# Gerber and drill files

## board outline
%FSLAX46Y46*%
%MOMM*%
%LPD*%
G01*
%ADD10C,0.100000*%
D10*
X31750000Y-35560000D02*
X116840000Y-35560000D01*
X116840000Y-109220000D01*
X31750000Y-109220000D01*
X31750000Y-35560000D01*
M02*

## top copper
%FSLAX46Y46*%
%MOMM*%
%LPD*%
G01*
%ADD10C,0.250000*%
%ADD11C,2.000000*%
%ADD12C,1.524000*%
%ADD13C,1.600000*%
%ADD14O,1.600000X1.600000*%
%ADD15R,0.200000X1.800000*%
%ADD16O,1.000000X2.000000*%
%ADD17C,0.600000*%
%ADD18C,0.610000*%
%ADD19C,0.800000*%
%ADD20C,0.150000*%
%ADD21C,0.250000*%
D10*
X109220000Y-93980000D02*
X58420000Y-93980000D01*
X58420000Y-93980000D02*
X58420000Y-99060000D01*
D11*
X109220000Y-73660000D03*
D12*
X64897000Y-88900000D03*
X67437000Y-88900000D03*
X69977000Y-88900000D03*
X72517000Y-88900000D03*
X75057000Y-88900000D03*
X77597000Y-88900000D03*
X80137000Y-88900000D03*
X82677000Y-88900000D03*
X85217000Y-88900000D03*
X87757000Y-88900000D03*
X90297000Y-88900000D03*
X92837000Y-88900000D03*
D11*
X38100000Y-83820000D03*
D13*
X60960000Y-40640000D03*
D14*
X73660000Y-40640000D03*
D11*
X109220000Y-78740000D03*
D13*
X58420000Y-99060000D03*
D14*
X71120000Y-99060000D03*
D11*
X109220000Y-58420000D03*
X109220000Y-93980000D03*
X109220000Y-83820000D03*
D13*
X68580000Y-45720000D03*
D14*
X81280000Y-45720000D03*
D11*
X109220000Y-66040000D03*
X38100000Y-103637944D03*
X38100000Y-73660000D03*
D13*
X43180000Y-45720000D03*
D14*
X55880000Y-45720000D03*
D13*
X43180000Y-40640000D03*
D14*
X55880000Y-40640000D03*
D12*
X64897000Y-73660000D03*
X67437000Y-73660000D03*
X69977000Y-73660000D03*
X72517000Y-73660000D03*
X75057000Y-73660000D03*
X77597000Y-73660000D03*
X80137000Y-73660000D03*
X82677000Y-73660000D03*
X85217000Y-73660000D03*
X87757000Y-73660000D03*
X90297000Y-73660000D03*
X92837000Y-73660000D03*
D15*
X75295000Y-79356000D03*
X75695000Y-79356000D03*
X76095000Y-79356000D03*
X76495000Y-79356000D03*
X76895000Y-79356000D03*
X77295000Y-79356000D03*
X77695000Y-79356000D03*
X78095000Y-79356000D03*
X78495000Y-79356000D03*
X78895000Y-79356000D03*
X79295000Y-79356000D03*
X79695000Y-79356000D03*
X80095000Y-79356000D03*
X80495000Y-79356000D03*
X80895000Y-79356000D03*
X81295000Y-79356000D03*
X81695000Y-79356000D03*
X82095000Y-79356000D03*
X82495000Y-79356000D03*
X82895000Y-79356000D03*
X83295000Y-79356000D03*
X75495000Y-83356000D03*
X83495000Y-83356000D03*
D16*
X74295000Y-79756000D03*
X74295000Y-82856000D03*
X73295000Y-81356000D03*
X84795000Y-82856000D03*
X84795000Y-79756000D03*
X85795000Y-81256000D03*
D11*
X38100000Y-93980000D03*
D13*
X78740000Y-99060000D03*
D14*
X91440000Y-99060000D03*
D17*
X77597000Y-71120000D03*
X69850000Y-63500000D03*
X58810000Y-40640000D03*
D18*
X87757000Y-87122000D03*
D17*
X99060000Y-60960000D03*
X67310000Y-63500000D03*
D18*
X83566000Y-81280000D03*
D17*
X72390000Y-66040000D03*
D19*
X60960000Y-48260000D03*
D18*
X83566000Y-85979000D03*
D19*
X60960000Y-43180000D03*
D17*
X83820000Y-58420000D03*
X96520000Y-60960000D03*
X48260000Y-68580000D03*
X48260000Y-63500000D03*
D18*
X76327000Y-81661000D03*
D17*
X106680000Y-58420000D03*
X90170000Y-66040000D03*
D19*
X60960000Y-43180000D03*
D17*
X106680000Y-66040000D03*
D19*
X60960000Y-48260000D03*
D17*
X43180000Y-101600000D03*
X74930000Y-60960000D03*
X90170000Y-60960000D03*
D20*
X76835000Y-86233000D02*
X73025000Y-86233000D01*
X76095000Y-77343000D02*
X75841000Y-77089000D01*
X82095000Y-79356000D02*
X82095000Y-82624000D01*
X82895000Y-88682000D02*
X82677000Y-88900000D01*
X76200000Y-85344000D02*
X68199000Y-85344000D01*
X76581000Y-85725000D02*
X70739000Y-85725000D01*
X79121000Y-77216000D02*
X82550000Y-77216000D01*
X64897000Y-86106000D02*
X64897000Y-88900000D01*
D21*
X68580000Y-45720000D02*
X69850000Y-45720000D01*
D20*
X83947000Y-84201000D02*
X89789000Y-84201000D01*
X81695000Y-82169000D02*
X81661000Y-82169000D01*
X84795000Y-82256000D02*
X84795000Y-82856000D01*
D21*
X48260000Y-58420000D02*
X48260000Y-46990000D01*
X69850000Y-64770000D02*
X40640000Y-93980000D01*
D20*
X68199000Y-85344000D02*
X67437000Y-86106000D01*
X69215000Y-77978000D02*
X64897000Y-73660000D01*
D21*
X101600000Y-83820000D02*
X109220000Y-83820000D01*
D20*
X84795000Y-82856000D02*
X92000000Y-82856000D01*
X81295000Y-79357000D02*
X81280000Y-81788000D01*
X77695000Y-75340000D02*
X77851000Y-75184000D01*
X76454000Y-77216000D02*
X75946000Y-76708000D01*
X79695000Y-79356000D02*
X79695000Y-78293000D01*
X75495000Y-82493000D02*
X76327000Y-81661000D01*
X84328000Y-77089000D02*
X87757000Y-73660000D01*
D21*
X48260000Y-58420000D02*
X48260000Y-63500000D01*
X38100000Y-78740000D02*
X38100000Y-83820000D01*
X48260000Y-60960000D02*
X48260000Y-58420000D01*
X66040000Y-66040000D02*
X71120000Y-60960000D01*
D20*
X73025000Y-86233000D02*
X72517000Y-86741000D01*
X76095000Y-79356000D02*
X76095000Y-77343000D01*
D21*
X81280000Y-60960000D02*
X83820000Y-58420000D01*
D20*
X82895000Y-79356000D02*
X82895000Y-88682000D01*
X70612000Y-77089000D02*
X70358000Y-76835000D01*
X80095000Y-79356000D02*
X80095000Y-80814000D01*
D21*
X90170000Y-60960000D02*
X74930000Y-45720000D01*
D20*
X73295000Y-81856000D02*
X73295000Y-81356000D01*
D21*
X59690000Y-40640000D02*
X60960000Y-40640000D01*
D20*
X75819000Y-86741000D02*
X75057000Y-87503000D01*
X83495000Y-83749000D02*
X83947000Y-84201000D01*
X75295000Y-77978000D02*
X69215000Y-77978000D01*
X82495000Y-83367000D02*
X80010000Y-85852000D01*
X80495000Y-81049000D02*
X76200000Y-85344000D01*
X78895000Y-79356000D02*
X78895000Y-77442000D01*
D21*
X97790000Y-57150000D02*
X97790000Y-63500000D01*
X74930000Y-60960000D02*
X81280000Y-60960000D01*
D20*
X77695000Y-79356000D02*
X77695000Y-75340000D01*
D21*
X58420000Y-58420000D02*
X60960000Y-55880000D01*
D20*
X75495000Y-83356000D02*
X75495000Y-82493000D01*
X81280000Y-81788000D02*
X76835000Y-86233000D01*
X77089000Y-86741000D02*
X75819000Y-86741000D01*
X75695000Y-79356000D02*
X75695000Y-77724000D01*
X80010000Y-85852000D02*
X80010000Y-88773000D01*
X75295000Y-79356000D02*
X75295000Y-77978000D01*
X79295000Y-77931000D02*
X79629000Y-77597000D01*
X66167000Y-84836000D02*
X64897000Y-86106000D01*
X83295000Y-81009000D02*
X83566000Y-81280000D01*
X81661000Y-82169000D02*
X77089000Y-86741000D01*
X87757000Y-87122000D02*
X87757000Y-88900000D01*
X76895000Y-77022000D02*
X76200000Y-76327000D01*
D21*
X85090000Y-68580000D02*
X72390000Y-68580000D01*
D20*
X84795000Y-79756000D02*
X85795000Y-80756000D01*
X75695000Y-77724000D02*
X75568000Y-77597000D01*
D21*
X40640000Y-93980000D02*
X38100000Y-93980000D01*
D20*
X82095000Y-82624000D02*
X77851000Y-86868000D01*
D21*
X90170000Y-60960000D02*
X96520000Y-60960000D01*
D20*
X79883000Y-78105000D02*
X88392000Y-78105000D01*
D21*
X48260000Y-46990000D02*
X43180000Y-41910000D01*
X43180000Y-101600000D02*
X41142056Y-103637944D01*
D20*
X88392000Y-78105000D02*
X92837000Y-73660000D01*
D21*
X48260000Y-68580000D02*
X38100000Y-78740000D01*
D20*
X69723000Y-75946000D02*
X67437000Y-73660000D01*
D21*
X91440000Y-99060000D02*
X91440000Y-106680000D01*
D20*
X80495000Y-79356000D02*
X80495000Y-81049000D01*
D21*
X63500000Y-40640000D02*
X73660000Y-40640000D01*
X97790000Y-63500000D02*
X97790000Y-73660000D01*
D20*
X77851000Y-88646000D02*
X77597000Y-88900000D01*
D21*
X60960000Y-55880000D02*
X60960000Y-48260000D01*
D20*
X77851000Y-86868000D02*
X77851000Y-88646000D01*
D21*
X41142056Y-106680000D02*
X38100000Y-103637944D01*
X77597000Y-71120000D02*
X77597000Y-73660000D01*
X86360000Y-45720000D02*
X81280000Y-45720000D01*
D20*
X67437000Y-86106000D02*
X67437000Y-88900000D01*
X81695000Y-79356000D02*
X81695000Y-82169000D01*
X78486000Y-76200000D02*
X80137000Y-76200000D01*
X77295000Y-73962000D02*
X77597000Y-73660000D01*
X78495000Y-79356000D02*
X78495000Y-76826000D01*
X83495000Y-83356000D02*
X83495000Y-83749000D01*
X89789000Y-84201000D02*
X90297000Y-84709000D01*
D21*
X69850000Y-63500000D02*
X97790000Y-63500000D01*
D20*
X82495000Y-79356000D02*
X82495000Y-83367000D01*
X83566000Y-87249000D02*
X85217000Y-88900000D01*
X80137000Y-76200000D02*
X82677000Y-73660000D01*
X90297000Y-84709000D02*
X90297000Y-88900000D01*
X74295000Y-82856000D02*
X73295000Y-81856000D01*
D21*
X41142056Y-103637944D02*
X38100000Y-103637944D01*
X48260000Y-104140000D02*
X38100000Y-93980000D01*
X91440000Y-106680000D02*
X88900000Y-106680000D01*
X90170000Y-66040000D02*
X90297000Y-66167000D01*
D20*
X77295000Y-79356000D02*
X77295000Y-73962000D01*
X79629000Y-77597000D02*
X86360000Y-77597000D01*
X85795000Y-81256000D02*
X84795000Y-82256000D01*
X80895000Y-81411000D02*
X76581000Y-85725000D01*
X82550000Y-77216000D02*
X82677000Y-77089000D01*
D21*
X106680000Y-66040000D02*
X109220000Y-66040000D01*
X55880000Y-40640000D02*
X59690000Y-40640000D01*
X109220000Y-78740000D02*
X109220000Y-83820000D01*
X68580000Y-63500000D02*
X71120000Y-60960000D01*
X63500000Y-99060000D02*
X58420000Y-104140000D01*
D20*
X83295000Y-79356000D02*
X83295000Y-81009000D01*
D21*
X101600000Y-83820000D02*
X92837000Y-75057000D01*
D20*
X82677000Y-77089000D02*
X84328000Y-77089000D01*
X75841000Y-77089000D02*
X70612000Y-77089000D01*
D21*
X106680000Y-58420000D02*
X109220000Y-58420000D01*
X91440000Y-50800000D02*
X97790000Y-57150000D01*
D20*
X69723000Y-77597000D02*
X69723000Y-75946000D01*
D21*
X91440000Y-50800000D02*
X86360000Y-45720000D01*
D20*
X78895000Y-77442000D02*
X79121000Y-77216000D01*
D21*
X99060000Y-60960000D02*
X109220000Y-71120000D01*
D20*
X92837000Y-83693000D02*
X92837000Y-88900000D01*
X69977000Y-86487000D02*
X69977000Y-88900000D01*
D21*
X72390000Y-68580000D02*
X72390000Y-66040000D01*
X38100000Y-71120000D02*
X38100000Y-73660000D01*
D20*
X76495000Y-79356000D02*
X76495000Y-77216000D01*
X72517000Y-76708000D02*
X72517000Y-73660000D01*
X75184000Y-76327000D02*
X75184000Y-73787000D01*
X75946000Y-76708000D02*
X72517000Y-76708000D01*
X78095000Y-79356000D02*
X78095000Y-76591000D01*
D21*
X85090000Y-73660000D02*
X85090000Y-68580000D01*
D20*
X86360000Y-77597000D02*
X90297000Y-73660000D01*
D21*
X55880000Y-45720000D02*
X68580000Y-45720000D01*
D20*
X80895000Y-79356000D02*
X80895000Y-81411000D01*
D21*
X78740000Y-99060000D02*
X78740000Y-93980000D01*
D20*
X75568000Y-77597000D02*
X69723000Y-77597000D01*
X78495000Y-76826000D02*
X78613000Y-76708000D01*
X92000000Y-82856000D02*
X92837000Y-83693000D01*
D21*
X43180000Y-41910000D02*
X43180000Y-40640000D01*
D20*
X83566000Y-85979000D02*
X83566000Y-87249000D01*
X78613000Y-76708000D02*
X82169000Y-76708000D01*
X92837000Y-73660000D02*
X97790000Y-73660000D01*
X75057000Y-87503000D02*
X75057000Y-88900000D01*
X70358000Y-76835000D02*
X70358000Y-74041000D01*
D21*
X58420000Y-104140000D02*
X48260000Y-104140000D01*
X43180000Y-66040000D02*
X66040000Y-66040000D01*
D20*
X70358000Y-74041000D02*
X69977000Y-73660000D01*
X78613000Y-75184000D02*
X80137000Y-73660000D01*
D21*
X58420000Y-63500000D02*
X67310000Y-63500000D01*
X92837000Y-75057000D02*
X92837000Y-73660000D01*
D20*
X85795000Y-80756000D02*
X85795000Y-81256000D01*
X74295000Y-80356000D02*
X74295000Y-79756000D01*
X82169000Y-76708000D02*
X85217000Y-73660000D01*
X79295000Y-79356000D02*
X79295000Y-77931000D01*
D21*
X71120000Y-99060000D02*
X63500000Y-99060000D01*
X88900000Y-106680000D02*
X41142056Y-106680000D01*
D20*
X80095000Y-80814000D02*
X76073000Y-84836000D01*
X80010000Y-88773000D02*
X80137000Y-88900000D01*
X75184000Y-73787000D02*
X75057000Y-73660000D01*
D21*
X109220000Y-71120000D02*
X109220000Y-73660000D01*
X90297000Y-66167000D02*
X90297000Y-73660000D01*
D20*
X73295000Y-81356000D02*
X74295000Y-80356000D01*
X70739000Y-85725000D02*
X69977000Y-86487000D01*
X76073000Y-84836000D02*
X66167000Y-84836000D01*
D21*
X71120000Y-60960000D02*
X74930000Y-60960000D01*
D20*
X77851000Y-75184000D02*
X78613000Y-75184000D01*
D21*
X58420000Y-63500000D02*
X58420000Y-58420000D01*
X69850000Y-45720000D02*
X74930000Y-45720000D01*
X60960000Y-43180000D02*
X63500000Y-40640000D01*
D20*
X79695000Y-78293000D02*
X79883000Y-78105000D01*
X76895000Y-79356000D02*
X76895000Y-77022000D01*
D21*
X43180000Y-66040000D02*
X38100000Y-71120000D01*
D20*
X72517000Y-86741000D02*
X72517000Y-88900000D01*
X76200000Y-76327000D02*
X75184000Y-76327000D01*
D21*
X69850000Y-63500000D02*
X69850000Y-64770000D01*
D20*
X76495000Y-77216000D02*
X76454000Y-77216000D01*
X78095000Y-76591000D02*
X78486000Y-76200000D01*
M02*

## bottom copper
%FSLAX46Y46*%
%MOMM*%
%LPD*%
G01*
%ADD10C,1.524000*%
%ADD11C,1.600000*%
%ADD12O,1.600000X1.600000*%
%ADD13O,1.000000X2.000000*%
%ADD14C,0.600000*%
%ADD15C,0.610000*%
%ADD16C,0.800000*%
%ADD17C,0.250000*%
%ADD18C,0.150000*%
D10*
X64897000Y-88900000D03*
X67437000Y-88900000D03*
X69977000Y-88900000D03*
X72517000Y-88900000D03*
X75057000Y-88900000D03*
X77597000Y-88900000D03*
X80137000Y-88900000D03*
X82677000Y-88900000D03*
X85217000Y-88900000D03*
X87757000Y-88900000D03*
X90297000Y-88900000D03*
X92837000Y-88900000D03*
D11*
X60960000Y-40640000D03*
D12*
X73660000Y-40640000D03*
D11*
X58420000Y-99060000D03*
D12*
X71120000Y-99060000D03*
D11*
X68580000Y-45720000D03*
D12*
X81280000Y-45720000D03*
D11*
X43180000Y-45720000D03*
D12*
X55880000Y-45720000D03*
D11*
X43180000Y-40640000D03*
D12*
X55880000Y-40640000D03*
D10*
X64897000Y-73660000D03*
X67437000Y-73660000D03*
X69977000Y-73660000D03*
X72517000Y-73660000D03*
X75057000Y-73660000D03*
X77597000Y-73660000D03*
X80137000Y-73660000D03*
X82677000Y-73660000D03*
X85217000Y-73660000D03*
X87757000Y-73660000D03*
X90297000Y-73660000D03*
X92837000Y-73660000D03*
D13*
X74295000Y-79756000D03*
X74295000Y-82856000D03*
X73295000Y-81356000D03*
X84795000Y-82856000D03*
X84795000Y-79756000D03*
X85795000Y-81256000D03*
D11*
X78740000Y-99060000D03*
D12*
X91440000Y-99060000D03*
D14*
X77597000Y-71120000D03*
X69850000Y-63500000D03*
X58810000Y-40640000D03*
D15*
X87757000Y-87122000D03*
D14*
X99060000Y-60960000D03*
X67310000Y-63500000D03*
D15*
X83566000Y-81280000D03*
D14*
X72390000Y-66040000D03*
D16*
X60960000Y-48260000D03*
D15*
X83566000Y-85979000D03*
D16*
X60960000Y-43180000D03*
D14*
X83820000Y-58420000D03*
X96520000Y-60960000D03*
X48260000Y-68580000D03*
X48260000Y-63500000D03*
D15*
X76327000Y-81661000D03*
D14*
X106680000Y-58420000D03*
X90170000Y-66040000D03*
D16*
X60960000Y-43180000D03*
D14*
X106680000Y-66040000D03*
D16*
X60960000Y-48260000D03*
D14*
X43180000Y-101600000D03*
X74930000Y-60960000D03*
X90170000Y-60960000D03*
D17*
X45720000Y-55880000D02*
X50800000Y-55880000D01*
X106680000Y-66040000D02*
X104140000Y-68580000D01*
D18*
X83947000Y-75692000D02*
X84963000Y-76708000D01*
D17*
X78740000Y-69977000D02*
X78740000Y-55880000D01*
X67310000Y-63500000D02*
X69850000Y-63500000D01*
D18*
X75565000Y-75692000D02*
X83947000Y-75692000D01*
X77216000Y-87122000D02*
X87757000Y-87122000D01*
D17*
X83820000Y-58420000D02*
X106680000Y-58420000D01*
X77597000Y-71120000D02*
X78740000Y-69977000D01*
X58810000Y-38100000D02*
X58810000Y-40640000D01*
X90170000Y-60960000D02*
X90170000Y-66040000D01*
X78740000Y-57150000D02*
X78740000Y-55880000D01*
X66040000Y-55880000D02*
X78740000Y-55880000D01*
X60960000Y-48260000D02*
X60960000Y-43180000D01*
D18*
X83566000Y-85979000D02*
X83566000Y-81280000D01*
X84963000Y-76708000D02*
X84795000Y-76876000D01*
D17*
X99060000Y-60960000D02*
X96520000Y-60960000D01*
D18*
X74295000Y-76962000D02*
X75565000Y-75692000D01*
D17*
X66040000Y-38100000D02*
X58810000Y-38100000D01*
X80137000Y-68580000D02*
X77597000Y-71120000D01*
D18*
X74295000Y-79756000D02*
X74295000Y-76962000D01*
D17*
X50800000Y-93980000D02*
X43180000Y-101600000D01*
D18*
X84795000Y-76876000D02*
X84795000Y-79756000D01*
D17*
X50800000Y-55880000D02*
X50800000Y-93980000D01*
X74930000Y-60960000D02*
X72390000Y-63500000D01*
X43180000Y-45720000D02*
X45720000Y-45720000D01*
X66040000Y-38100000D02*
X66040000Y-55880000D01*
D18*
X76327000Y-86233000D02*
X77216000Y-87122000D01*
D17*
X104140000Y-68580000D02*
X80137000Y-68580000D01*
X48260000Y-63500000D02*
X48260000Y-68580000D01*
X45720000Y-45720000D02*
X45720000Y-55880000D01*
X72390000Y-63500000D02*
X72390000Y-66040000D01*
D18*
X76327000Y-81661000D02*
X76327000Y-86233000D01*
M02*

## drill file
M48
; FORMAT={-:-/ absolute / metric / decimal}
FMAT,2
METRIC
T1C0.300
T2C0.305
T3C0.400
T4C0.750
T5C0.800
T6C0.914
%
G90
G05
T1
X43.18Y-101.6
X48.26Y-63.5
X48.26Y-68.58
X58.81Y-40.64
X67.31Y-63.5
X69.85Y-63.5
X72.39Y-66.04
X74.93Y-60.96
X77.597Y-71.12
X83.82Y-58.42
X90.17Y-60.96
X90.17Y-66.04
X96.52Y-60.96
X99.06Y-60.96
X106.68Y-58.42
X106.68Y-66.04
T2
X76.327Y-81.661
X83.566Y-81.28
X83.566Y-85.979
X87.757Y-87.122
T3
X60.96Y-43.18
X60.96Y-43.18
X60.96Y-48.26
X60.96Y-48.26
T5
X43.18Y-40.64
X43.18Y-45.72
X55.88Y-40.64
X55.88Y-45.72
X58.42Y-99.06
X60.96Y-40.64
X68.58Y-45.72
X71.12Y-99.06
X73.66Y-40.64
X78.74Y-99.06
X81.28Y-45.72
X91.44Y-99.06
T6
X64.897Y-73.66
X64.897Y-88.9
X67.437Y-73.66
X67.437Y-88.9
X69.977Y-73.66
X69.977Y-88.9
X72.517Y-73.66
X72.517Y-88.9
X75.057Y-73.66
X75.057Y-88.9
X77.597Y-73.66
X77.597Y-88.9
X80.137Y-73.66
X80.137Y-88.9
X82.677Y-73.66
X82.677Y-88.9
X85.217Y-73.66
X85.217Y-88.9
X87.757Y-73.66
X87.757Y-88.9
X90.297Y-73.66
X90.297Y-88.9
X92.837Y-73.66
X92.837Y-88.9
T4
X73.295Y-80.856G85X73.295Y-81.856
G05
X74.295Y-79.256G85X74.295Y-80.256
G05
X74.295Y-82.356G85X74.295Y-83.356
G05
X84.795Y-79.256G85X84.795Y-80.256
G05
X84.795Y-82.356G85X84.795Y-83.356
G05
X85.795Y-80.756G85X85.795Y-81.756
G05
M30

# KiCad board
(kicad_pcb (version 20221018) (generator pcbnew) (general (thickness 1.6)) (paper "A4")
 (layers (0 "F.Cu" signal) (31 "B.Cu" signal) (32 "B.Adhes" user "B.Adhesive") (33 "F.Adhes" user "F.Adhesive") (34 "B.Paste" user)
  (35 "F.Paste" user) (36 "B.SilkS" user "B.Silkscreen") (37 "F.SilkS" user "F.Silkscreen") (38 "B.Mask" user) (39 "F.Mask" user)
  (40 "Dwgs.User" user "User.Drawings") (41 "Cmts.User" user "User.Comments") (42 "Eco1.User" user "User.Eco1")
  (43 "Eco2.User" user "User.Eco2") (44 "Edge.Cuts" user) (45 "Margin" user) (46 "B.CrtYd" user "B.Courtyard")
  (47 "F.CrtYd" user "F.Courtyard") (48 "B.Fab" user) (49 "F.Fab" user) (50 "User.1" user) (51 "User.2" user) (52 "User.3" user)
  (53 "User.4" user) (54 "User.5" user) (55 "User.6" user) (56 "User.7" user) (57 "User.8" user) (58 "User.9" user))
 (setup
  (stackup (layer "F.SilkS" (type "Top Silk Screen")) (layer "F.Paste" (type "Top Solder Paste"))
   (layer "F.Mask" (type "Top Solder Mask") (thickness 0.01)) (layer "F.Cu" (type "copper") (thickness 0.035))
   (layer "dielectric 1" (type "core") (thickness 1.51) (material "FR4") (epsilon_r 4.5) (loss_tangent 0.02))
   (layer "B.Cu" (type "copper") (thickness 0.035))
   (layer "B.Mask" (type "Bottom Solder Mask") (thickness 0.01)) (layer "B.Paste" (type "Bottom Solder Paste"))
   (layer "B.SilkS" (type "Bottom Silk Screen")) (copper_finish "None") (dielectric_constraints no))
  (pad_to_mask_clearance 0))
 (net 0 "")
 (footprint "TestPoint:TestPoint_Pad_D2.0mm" (layer "F.Cu") (at 109.22 73.66)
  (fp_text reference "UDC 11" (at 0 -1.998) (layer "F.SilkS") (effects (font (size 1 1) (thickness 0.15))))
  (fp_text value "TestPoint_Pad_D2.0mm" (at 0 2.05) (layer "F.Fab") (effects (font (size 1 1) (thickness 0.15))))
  (pad "7" smd circle (at 0 0) (size 2 2) (layers "F.Cu" "F.Mask")))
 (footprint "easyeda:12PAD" (layer "F.Cu") (at 64.897 88.9)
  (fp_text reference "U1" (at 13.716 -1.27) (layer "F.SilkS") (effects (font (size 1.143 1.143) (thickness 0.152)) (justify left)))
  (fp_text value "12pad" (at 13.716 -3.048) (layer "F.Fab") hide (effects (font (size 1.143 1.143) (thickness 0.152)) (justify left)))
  (pad "1" thru_hole circle (at 0 0) (size 1.524 1.524) (drill 0.914) (layers "*.Cu" "*.Paste" "*.Mask"))
  (pad "2" thru_hole circle (at 2.54 0) (size 1.524 1.524) (drill 0.914) (layers "*.Cu" "*.Paste" "*.Mask"))
  (pad "3" thru_hole circle (at 5.08 0) (size 1.524 1.524) (drill 0.914) (layers "*.Cu" "*.Paste" "*.Mask"))
  (pad "4" thru_hole circle (at 7.62 0) (size 1.524 1.524) (drill 0.914) (layers "*.Cu" "*.Paste" "*.Mask"))
  (pad "5" thru_hole circle (at 10.16 0) (size 1.524 1.524) (drill 0.914) (layers "*.Cu" "*.Paste" "*.Mask"))
  (pad "6" thru_hole circle (at 12.7 0) (size 1.524 1.524) (drill 0.914) (layers "*.Cu" "*.Paste" "*.Mask"))
  (pad "7" thru_hole circle (at 15.24 0) (size 1.524 1.524) (drill 0.914) (layers "*.Cu" "*.Paste" "*.Mask"))
  (pad "8" thru_hole circle (at 17.78 0) (size 1.524 1.524) (drill 0.914) (layers "*.Cu" "*.Paste" "*.Mask"))
  (pad "9" thru_hole circle (at 20.32 0) (size 1.524 1.524) (drill 0.914) (layers "*.Cu" "*.Paste" "*.Mask"))
  (pad "10" thru_hole circle (at 22.86 0) (size 1.524 1.524) (drill 0.914) (layers "*.Cu" "*.Paste" "*.Mask"))
  (pad "11" thru_hole circle (at 25.4 0) (size 1.524 1.524) (drill 0.914) (layers "*.Cu" "*.Paste" "*.Mask"))
  (pad "12" thru_hole circle (at 27.94 0) (size 1.524 1.524) (drill 0.914) (layers "*.Cu" "*.Paste" "*.Mask")))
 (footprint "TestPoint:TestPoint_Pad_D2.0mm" (layer "F.Cu") (at 38.1 83.82)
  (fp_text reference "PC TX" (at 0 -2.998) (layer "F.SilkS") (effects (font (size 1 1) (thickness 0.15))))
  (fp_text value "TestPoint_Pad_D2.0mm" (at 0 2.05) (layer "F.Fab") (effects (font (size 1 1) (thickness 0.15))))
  (pad "2" smd circle (at 0 0) (size 2 2) (layers "F.Cu" "F.Mask")))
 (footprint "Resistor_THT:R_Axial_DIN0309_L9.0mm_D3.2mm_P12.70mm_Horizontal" (layer "F.Cu") (at 60.96 40.64)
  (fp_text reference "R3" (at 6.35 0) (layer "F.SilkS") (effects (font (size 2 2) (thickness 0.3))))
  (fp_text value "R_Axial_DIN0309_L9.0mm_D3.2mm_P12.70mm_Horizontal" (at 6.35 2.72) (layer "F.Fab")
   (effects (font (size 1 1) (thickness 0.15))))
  (pad "1" thru_hole circle (at 0 0) (size 1.6 1.6) (drill 0.8) (layers "*.Cu" "*.Mask"))
  (pad "2" thru_hole oval (at 12.7 0) (size 1.6 1.6) (drill 0.8) (layers "*.Cu" "*.Mask")))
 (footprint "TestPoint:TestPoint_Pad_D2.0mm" (layer "F.Cu") (at 109.22 78.74)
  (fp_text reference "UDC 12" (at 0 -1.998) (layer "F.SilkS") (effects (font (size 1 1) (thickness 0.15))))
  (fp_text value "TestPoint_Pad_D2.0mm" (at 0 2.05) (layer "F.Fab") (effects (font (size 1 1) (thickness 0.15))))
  (pad "8" smd circle (at 0 0) (size 2 2) (layers "F.Cu" "F.Mask")))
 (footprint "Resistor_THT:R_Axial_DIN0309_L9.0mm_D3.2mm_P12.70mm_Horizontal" (layer "F.Cu") (at 58.42 99.06)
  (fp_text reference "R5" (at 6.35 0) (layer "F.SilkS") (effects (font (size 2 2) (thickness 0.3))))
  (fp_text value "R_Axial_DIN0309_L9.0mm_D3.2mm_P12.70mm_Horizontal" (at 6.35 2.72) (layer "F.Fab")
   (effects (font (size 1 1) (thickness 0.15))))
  (pad "1" thru_hole circle (at 0 0) (size 1.6 1.6) (drill 0.8) (layers "*.Cu" "*.Mask"))
  (pad "2" thru_hole oval (at 12.7 0) (size 1.6 1.6) (drill 0.8) (layers "*.Cu" "*.Mask")))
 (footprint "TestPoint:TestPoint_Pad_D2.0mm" (layer "F.Cu") (at 109.22 58.42)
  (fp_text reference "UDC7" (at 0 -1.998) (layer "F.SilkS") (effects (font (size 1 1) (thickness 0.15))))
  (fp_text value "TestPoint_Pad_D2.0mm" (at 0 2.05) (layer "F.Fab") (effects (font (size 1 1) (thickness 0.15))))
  (pad "5" smd circle (at 0 0) (size 2 2) (layers "F.Cu" "F.Mask")))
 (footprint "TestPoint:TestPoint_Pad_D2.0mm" (layer "F.Cu") (at 109.22 93.98)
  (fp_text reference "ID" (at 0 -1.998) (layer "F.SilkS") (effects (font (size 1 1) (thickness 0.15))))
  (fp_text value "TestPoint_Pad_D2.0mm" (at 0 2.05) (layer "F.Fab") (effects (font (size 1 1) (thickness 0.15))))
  (pad "9" smd circle (at 0 0) (size 2 2) (layers "F.Cu" "F.Mask")))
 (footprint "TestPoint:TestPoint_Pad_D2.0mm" (layer "F.Cu") (at 109.22 83.82)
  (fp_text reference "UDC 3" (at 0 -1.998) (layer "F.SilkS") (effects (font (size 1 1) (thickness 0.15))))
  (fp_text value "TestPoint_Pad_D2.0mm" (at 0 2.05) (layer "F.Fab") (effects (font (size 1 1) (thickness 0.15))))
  (pad "9" smd circle (at 0 0) (size 2 2) (layers "F.Cu" "F.Mask")))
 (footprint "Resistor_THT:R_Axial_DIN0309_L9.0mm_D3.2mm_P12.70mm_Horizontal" (layer "F.Cu") (at 68.58 45.72)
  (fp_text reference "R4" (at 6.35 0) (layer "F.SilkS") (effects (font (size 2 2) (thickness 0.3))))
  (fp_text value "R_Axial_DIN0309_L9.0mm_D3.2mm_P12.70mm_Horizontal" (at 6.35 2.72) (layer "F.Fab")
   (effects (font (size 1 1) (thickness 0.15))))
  (pad "1" thru_hole circle (at 0 0) (size 1.6 1.6) (drill 0.8) (layers "*.Cu" "*.Mask"))
  (pad "2" thru_hole oval (at 12.7 0) (size 1.6 1.6) (drill 0.8) (layers "*.Cu" "*.Mask")))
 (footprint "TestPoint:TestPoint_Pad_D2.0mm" (layer "F.Cu") (at 109.22 66.04)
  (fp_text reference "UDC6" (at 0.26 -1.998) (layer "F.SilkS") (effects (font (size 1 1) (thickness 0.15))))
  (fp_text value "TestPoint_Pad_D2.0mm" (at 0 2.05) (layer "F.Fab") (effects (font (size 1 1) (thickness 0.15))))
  (pad "6" smd circle (at 0 0) (size 2 2) (layers "F.Cu" "F.Mask")))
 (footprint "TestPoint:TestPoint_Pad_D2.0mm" (layer "F.Cu") (at 38.1 103.637944)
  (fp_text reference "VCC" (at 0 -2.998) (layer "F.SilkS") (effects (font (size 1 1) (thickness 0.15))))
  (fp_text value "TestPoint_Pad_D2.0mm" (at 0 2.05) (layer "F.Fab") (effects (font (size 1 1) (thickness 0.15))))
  (pad "4" smd circle (at 0 0) (size 2 2) (layers "F.Cu" "F.Mask")))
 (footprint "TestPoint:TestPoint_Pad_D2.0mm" (layer "F.Cu") (at 38.1 73.66)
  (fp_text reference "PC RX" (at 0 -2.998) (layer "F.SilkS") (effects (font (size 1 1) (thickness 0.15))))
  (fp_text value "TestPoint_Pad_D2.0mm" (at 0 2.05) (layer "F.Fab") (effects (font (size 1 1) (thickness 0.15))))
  (pad "1" smd circle (at 0 0) (size 2 2) (layers "F.Cu" "F.Mask")))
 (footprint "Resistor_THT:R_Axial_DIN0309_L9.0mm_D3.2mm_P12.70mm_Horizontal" (layer "F.Cu") (at 43.18 45.72)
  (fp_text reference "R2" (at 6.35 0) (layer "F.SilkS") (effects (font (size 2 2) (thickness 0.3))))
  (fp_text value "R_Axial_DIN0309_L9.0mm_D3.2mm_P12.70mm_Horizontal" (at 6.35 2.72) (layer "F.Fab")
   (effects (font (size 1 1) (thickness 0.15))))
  (pad "1" thru_hole circle (at 0 0) (size 1.6 1.6) (drill 0.8) (layers "*.Cu" "*.Mask"))
  (pad "2" thru_hole oval (at 12.7 0) (size 1.6 1.6) (drill 0.8) (layers "*.Cu" "*.Mask")))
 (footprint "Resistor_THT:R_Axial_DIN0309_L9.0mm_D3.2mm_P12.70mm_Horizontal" (layer "F.Cu") (at 43.18 40.64)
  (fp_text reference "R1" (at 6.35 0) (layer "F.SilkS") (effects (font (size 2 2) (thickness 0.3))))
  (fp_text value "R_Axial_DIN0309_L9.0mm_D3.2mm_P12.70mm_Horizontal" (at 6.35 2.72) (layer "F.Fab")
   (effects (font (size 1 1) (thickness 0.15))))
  (pad "1" thru_hole circle (at 0 0) (size 1.6 1.6) (drill 0.8) (layers "*.Cu" "*.Mask"))
  (pad "2" thru_hole oval (at 12.7 0) (size 1.6 1.6) (drill 0.8) (layers "*.Cu" "*.Mask")))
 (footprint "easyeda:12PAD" (layer "F.Cu") (at 64.897 73.66)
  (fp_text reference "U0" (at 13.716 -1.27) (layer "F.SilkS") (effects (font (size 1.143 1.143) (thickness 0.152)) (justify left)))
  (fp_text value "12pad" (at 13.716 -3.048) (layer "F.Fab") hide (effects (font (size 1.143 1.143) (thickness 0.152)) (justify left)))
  (pad "1" thru_hole circle (at 0 0) (size 1.524 1.524) (drill 0.914) (layers "*.Cu" "*.Paste" "*.Mask"))
  (pad "2" thru_hole circle (at 2.54 0) (size 1.524 1.524) (drill 0.914) (layers "*.Cu" "*.Paste" "*.Mask"))
  (pad "3" thru_hole circle (at 5.08 0) (size 1.524 1.524) (drill 0.914) (layers "*.Cu" "*.Paste" "*.Mask"))
  (pad "4" thru_hole circle (at 7.62 0) (size 1.524 1.524) (drill 0.914) (layers "*.Cu" "*.Paste" "*.Mask"))
  (pad "5" thru_hole circle (at 10.16 0) (size 1.524 1.524) (drill 0.914) (layers "*.Cu" "*.Paste" "*.Mask"))
  (pad "6" thru_hole circle (at 12.7 0) (size 1.524 1.524) (drill 0.914) (layers "*.Cu" "*.Paste" "*.Mask"))
  (pad "7" thru_hole circle (at 15.24 0) (size 1.524 1.524) (drill 0.914) (layers "*.Cu" "*.Paste" "*.Mask"))
  (pad "8" thru_hole circle (at 17.78 0) (size 1.524 1.524) (drill 0.914) (layers "*.Cu" "*.Paste" "*.Mask"))
  (pad "9" thru_hole circle (at 20.32 0) (size 1.524 1.524) (drill 0.914) (layers "*.Cu" "*.Paste" "*.Mask"))
  (pad "10" thru_hole circle (at 22.86 0) (size 1.524 1.524) (drill 0.914) (layers "*.Cu" "*.Paste" "*.Mask"))
  (pad "11" thru_hole circle (at 25.4 0) (size 1.524 1.524) (drill 0.914) (layers "*.Cu" "*.Paste" "*.Mask"))
  (pad "12" thru_hole circle (at 27.94 0) (size 1.524 1.524) (drill 0.914) (layers "*.Cu" "*.Paste" "*.Mask")))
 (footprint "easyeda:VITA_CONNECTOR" (layer "F.Cu") (at 74.295 79.756)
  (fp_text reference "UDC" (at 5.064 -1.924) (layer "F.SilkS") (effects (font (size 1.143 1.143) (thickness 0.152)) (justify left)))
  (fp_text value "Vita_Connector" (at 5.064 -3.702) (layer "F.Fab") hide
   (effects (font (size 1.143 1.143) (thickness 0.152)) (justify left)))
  (pad "1" smd rect (at 1 -0.4) (size 0.2 1.8) (layers "F.Cu" "F.Paste" "F.Mask"))
  (pad "2" smd rect (at 1.4 -0.4) (size 0.2 1.8) (layers "F.Cu" "F.Paste" "F.Mask"))
  (pad "3" smd rect (at 1.8 -0.4) (size 0.2 1.8) (layers "F.Cu" "F.Paste" "F.Mask"))
  (pad "4" smd rect (at 2.2 -0.4) (size 0.2 1.8) (layers "F.Cu" "F.Paste" "F.Mask"))
  (pad "5" smd rect (at 2.6 -0.4) (size 0.2 1.8) (layers "F.Cu" "F.Paste" "F.Mask"))
  (pad "6" smd rect (at 3 -0.4) (size 0.2 1.8) (layers "F.Cu" "F.Paste" "F.Mask"))
  (pad "7" smd rect (at 3.4 -0.4) (size 0.2 1.8) (layers "F.Cu" "F.Paste" "F.Mask"))
  (pad "8" smd rect (at 3.8 -0.4) (size 0.2 1.8) (layers "F.Cu" "F.Paste" "F.Mask"))
  (pad "9" smd rect (at 4.2 -0.4) (size 0.2 1.8) (layers "F.Cu" "F.Paste" "F.Mask"))
  (pad "10" smd rect (at 4.6 -0.4) (size 0.2 1.8) (layers "F.Cu" "F.Paste" "F.Mask"))
  (pad "11" smd rect (at 5 -0.4) (size 0.2 1.8) (layers "F.Cu" "F.Paste" "F.Mask"))
  (pad "12" smd rect (at 5.4 -0.4) (size 0.2 1.8) (layers "F.Cu" "F.Paste" "F.Mask"))
  (pad "13" smd rect (at 5.8 -0.4) (size 0.2 1.8) (layers "F.Cu" "F.Paste" "F.Mask"))
  (pad "14" smd rect (at 6.2 -0.4) (size 0.2 1.8) (layers "F.Cu" "F.Paste" "F.Mask"))
  (pad "15" smd rect (at 6.6 -0.4) (size 0.2 1.8) (layers "F.Cu" "F.Paste" "F.Mask"))
  (pad "16" smd rect (at 7 -0.4) (size 0.2 1.8) (layers "F.Cu" "F.Paste" "F.Mask"))
  (pad "17" smd rect (at 7.4 -0.4) (size 0.2 1.8) (layers "F.Cu" "F.Paste" "F.Mask"))
  (pad "18" smd rect (at 7.8 -0.4) (size 0.2 1.8) (layers "F.Cu" "F.Paste" "F.Mask"))
  (pad "19" smd rect (at 8.2 -0.4) (size 0.2 1.8) (layers "F.Cu" "F.Paste" "F.Mask"))
  (pad "20" smd rect (at 8.6 -0.4) (size 0.2 1.8) (layers "F.Cu" "F.Paste" "F.Mask"))
  (pad "21" smd rect (at 9 -0.4) (size 0.2 1.8) (layers "F.Cu" "F.Paste" "F.Mask"))
  (pad "22" smd rect (at 1.2 3.6) (size 0.2 1.8) (layers "F.Cu" "F.Paste" "F.Mask"))
  (pad "23" smd rect (at 9.2 3.6) (size 0.2 1.8) (layers "F.Cu" "F.Paste" "F.Mask"))
  (pad "24" thru_hole oval (at 0 0) (size 1 2) (drill oval 0.75 1.75) (layers "*.Cu" "*.Paste" "*.Mask"))
  (pad "25" thru_hole oval (at 0 3.1) (size 1 2) (drill oval 0.75 1.75) (layers "*.Cu" "*.Paste" "*.Mask"))
  (pad "26" thru_hole oval (at -1 1.6) (size 1 2) (drill oval 0.75 1.75) (layers "*.Cu" "*.Paste" "*.Mask"))
  (pad "27" thru_hole oval (at 10.5 3.1) (size 1 2) (drill oval 0.75 1.75) (layers "*.Cu" "*.Paste" "*.Mask"))
  (pad "28" thru_hole oval (at 10.5 0) (size 1 2) (drill oval 0.75 1.75) (layers "*.Cu" "*.Paste" "*.Mask"))
  (pad "29" thru_hole oval (at 11.5 1.5) (size 1 2) (drill oval 0.75 1.75) (layers "*.Cu" "*.Paste" "*.Mask")))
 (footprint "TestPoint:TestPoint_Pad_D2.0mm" (layer "F.Cu") (at 38.1 93.98)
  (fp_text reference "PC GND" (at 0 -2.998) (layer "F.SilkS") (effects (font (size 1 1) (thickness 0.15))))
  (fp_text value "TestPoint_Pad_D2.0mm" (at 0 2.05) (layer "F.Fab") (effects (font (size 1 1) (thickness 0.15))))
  (pad "3" smd circle (at 0 0) (size 2 2) (layers "F.Cu" "F.Mask")))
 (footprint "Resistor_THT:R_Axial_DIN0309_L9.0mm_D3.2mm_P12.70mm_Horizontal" (layer "F.Cu") (at 78.74 99.06)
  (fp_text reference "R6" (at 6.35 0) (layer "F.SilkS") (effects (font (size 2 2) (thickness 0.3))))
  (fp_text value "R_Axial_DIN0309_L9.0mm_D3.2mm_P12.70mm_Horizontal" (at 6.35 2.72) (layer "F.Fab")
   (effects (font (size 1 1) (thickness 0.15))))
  (pad "1" thru_hole circle (at 0 0) (size 1.6 1.6) (drill 0.8) (layers "*.Cu" "*.Mask"))
  (pad "2" thru_hole oval (at 12.7 0) (size 1.6 1.6) (drill 0.8) (layers "*.Cu" "*.Mask")))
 (gr_line (start 109.22 93.98) (end 58.42 93.98) (stroke (width 0.25) (type default)) (layer "F.Cu"))
 (gr_line (start 58.42 93.98) (end 58.42 99.06) (stroke (width 0.25) (type default)) (layer "F.Cu"))
 (gr_rect (start 31.75 35.56) (end 116.84 109.22) (stroke (width 0.1) (type default)) (fill none) (layer "Edge.Cuts"))
 (segment (start 76.835 86.233) (end 73.025 86.233) (width 0.15) (layer "F.Cu") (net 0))
 (segment (start 76.095 77.343) (end 75.841 77.089) (width 0.15) (layer "F.Cu") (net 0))
 (segment (start 82.095 79.356) (end 82.095 82.624) (width 0.15) (layer "F.Cu") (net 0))
 (segment (start 82.895 88.682) (end 82.677 88.9) (width 0.15) (layer "F.Cu") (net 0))
 (segment (start 76.2 85.344) (end 68.199 85.344) (width 0.15) (layer "F.Cu") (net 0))
 (segment (start 76.581 85.725) (end 70.739 85.725) (width 0.15) (layer "F.Cu") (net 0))
 (segment (start 79.121 77.216) (end 82.55 77.216) (width 0.15) (layer "F.Cu") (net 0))
 (segment (start 64.897 86.106) (end 64.897 88.9) (width 0.15) (layer "F.Cu") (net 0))
 (segment (start 68.58 45.72) (end 69.85 45.72) (width 0.25) (layer "F.Cu") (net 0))
 (segment (start 83.947 84.201) (end 89.789 84.201) (width 0.15) (layer "F.Cu") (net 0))
 (segment (start 81.695 82.169) (end 81.661 82.169) (width 0.15) (layer "F.Cu") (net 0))
 (segment (start 84.795 82.256) (end 84.795 82.856) (width 0.15) (layer "F.Cu") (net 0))
 (segment (start 48.26 58.42) (end 48.26 46.99) (width 0.25) (layer "F.Cu") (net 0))
 (segment (start 69.85 64.77) (end 40.64 93.98) (width 0.25) (layer "F.Cu") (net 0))
 (segment (start 68.199 85.344) (end 67.437 86.106) (width 0.15) (layer "F.Cu") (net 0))
 (segment (start 69.215 77.978) (end 64.897 73.66) (width 0.15) (layer "F.Cu") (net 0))
 (segment (start 101.6 83.82) (end 109.22 83.82) (width 0.25) (layer "F.Cu") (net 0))
 (segment (start 84.795 82.856) (end 92 82.856) (width 0.15) (layer "F.Cu") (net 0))
 (segment (start 81.295 79.357) (end 81.28 81.788) (width 0.15) (layer "F.Cu") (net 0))
 (segment (start 77.695 75.34) (end 77.851 75.184) (width 0.15) (layer "F.Cu") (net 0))
 (segment (start 76.454 77.216) (end 75.946 76.708) (width 0.15) (layer "F.Cu") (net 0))
 (segment (start 79.695 79.356) (end 79.695 78.293) (width 0.15) (layer "F.Cu") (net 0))
 (segment (start 75.495 82.493) (end 76.327 81.661) (width 0.15) (layer "F.Cu") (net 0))
 (segment (start 84.328 77.089) (end 87.757 73.66) (width 0.15) (layer "F.Cu") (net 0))
 (segment (start 48.26 58.42) (end 48.26 63.5) (width 0.25) (layer "F.Cu") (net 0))
 (segment (start 38.1 78.74) (end 38.1 83.82) (width 0.25) (layer "F.Cu") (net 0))
 (segment (start 48.26 60.96) (end 48.26 58.42) (width 0.25) (layer "F.Cu") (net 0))
 (segment (start 66.04 66.04) (end 71.12 60.96) (width 0.25) (layer "F.Cu") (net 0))
 (segment (start 73.025 86.233) (end 72.517 86.741) (width 0.15) (layer "F.Cu") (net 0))
 (segment (start 76.095 79.356) (end 76.095 77.343) (width 0.15) (layer "F.Cu") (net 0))
 (segment (start 81.28 60.96) (end 83.82 58.42) (width 0.25) (layer "F.Cu") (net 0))
 (segment (start 82.895 79.356) (end 82.895 88.682) (width 0.15) (layer "F.Cu") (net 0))
 (segment (start 70.612 77.089) (end 70.358 76.835) (width 0.15) (layer "F.Cu") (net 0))
 (segment (start 80.095 79.356) (end 80.095 80.814) (width 0.15) (layer "F.Cu") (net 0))
 (segment (start 90.17 60.96) (end 74.93 45.72) (width 0.25) (layer "F.Cu") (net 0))
 (segment (start 73.295 81.856) (end 73.295 81.356) (width 0.15) (layer "F.Cu") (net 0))
 (segment (start 59.69 40.64) (end 60.96 40.64) (width 0.25) (layer "F.Cu") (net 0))
 (segment (start 75.819 86.741) (end 75.057 87.503) (width 0.15) (layer "F.Cu") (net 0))
 (segment (start 83.495 83.749) (end 83.947 84.201) (width 0.15) (layer "F.Cu") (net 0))
 (segment (start 75.295 77.978) (end 69.215 77.978) (width 0.15) (layer "F.Cu") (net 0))
 (segment (start 82.495 83.367) (end 80.01 85.852) (width 0.15) (layer "F.Cu") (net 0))
 (segment (start 80.495 81.049) (end 76.2 85.344) (width 0.15) (layer "F.Cu") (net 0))
 (segment (start 78.895 79.356) (end 78.895 77.442) (width 0.15) (layer "F.Cu") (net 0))
 (segment (start 97.79 57.15) (end 97.79 63.5) (width 0.25) (layer "F.Cu") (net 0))
 (segment (start 74.93 60.96) (end 81.28 60.96) (width 0.25) (layer "F.Cu") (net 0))
 (segment (start 77.695 79.356) (end 77.695 75.34) (width 0.15) (layer "F.Cu") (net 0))
 (segment (start 58.42 58.42) (end 60.96 55.88) (width 0.25) (layer "F.Cu") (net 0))
 (segment (start 75.495 83.356) (end 75.495 82.493) (width 0.15) (layer "F.Cu") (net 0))
 (segment (start 81.28 81.788) (end 76.835 86.233) (width 0.15) (layer "F.Cu") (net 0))
 (segment (start 77.089 86.741) (end 75.819 86.741) (width 0.15) (layer "F.Cu") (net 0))
 (segment (start 75.695 79.356) (end 75.695 77.724) (width 0.15) (layer "F.Cu") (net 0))
 (segment (start 80.01 85.852) (end 80.01 88.773) (width 0.15) (layer "F.Cu") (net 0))
 (segment (start 75.295 79.356) (end 75.295 77.978) (width 0.15) (layer "F.Cu") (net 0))
 (segment (start 79.295 77.931) (end 79.629 77.597) (width 0.15) (layer "F.Cu") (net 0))
 (segment (start 66.167 84.836) (end 64.897 86.106) (width 0.15) (layer "F.Cu") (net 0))
 (segment (start 83.295 81.009) (end 83.566 81.28) (width 0.15) (layer "F.Cu") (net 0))
 (segment (start 81.661 82.169) (end 77.089 86.741) (width 0.15) (layer "F.Cu") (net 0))
 (segment (start 87.757 87.122) (end 87.757 88.9) (width 0.15) (layer "F.Cu") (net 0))
 (segment (start 76.895 77.022) (end 76.2 76.327) (width 0.15) (layer "F.Cu") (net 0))
 (segment (start 85.09 68.58) (end 72.39 68.58) (width 0.25) (layer "F.Cu") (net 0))
 (segment (start 84.795 79.756) (end 85.795 80.756) (width 0.15) (layer "F.Cu") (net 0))
 (segment (start 75.695 77.724) (end 75.568 77.597) (width 0.15) (layer "F.Cu") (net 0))
 (segment (start 40.64 93.98) (end 38.1 93.98) (width 0.25) (layer "F.Cu") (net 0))
 (segment (start 82.095 82.624) (end 77.851 86.868) (width 0.15) (layer "F.Cu") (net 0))
 (segment (start 90.17 60.96) (end 96.52 60.96) (width 0.25) (layer "F.Cu") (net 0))
 (segment (start 79.883 78.105) (end 88.392 78.105) (width 0.15) (layer "F.Cu") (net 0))
 (segment (start 48.26 46.99) (end 43.18 41.91) (width 0.25) (layer "F.Cu") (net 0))
 (segment (start 43.18 101.6) (end 41.142056 103.637944) (width 0.25) (layer "F.Cu") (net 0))
 (segment (start 88.392 78.105) (end 92.837 73.66) (width 0.15) (layer "F.Cu") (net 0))
 (segment (start 48.26 68.58) (end 38.1 78.74) (width 0.25) (layer "F.Cu") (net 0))
 (segment (start 69.723 75.946) (end 67.437 73.66) (width 0.15) (layer "F.Cu") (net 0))
 (segment (start 91.44 99.06) (end 91.44 106.68) (width 0.25) (layer "F.Cu") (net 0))
 (segment (start 80.495 79.356) (end 80.495 81.049) (width 0.15) (layer "F.Cu") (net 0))
 (segment (start 63.5 40.64) (end 73.66 40.64) (width 0.25) (layer "F.Cu") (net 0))
 (segment (start 97.79 63.5) (end 97.79 73.66) (width 0.25) (layer "F.Cu") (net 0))
 (segment (start 77.851 88.646) (end 77.597 88.9) (width 0.15) (layer "F.Cu") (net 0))
 (segment (start 60.96 55.88) (end 60.96 48.26) (width 0.25) (layer "F.Cu") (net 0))
 (segment (start 77.851 86.868) (end 77.851 88.646) (width 0.15) (layer "F.Cu") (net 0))
 (segment (start 41.142056 106.68) (end 38.1 103.637944) (width 0.25) (layer "F.Cu") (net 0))
 (segment (start 77.597 71.12) (end 77.597 73.66) (width 0.25) (layer "F.Cu") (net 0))
 (segment (start 86.36 45.72) (end 81.28 45.72) (width 0.25) (layer "F.Cu") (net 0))
 (segment (start 67.437 86.106) (end 67.437 88.9) (width 0.15) (layer "F.Cu") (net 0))
 (segment (start 81.695 79.356) (end 81.695 82.169) (width 0.15) (layer "F.Cu") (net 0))
 (segment (start 78.486 76.2) (end 80.137 76.2) (width 0.15) (layer "F.Cu") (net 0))
 (segment (start 77.295 73.962) (end 77.597 73.66) (width 0.15) (layer "F.Cu") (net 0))
 (segment (start 78.495 79.356) (end 78.495 76.826) (width 0.15) (layer "F.Cu") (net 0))
 (segment (start 83.495 83.356) (end 83.495 83.749) (width 0.15) (layer "F.Cu") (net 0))
 (segment (start 89.789 84.201) (end 90.297 84.709) (width 0.15) (layer "F.Cu") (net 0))
 (segment (start 69.85 63.5) (end 97.79 63.5) (width 0.25) (layer "F.Cu") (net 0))
 (segment (start 82.495 79.356) (end 82.495 83.367) (width 0.15) (layer "F.Cu") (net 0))
 (segment (start 83.566 87.249) (end 85.217 88.9) (width 0.15) (layer "F.Cu") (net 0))
 (segment (start 80.137 76.2) (end 82.677 73.66) (width 0.15) (layer "F.Cu") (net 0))
 (segment (start 90.297 84.709) (end 90.297 88.9) (width 0.15) (layer "F.Cu") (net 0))
 (segment (start 74.295 82.856) (end 73.295 81.856) (width 0.15) (layer "F.Cu") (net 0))
 (segment (start 41.142056 103.637944) (end 38.1 103.637944) (width 0.25) (layer "F.Cu") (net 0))
 (segment (start 48.26 104.14) (end 38.1 93.98) (width 0.25) (layer "F.Cu") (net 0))
 (segment (start 91.44 106.68) (end 88.9 106.68) (width 0.25) (layer "F.Cu") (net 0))
 (segment (start 90.17 66.04) (end 90.297 66.167) (width 0.25) (layer "F.Cu") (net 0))
 (segment (start 77.295 79.356) (end 77.295 73.962) (width 0.15) (layer "F.Cu") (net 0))
 (segment (start 79.629 77.597) (end 86.36 77.597) (width 0.15) (layer "F.Cu") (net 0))
 (segment (start 85.795 81.256) (end 84.795 82.256) (width 0.15) (layer "F.Cu") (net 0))
 (segment (start 80.895 81.411) (end 76.581 85.725) (width 0.15) (layer "F.Cu") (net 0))
 (segment (start 82.55 77.216) (end 82.677 77.089) (width 0.15) (layer "F.Cu") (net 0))
 (segment (start 106.68 66.04) (end 109.22 66.04) (width 0.25) (layer "F.Cu") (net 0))
 (segment (start 55.88 40.64) (end 59.69 40.64) (width 0.25) (layer "F.Cu") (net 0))
 (segment (start 109.22 78.74) (end 109.22 83.82) (width 0.25) (layer "F.Cu") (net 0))
 (segment (start 68.58 63.5) (end 71.12 60.96) (width 0.25) (layer "F.Cu") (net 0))
 (segment (start 63.5 99.06) (end 58.42 104.14) (width 0.25) (layer "F.Cu") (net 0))
 (segment (start 83.295 79.356) (end 83.295 81.009) (width 0.15) (layer "F.Cu") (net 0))
 (segment (start 101.6 83.82) (end 92.837 75.057) (width 0.25) (layer "F.Cu") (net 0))
 (segment (start 82.677 77.089) (end 84.328 77.089) (width 0.15) (layer "F.Cu") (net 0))
 (segment (start 75.841 77.089) (end 70.612 77.089) (width 0.15) (layer "F.Cu") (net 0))
 (segment (start 106.68 58.42) (end 109.22 58.42) (width 0.25) (layer "F.Cu") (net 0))
 (segment (start 91.44 50.8) (end 97.79 57.15) (width 0.25) (layer "F.Cu") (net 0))
 (segment (start 69.723 77.597) (end 69.723 75.946) (width 0.15) (layer "F.Cu") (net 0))
 (segment (start 91.44 50.8) (end 86.36 45.72) (width 0.25) (layer "F.Cu") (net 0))
 (segment (start 78.895 77.442) (end 79.121 77.216) (width 0.15) (layer "F.Cu") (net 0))
 (segment (start 99.06 60.96) (end 109.22 71.12) (width 0.25) (layer "F.Cu") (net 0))
 (segment (start 92.837 83.693) (end 92.837 88.9) (width 0.15) (layer "F.Cu") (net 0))
 (segment (start 69.977 86.487) (end 69.977 88.9) (width 0.15) (layer "F.Cu") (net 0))
 (segment (start 72.39 68.58) (end 72.39 66.04) (width 0.25) (layer "F.Cu") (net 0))
 (segment (start 38.1 71.12) (end 38.1 73.66) (width 0.25) (layer "F.Cu") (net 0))
 (segment (start 76.495 79.356) (end 76.495 77.216) (width 0.15) (layer "F.Cu") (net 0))
 (segment (start 72.517 76.708) (end 72.517 73.66) (width 0.15) (layer "F.Cu") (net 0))
 (segment (start 75.184 76.327) (end 75.184 73.787) (width 0.15) (layer "F.Cu") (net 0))
 (segment (start 75.946 76.708) (end 72.517 76.708) (width 0.15) (layer "F.Cu") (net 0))
 (segment (start 78.095 79.356) (end 78.095 76.591) (width 0.15) (layer "F.Cu") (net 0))
 (segment (start 85.09 73.66) (end 85.09 68.58) (width 0.25) (layer "F.Cu") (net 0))
 (segment (start 86.36 77.597) (end 90.297 73.66) (width 0.15) (layer "F.Cu") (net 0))
 (segment (start 55.88 45.72) (end 68.58 45.72) (width 0.25) (layer "F.Cu") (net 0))
 (segment (start 80.895 79.356) (end 80.895 81.411) (width 0.15) (layer "F.Cu") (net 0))
 (segment (start 78.74 99.06) (end 78.74 93.98) (width 0.25) (layer "F.Cu") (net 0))
 (segment (start 75.568 77.597) (end 69.723 77.597) (width 0.15) (layer "F.Cu") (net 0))
 (segment (start 78.495 76.826) (end 78.613 76.708) (width 0.15) (layer "F.Cu") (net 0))
 (segment (start 92 82.856) (end 92.837 83.693) (width 0.15) (layer "F.Cu") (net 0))
 (segment (start 43.18 41.91) (end 43.18 40.64) (width 0.25) (layer "F.Cu") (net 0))
 (segment (start 83.566 85.979) (end 83.566 87.249) (width 0.15) (layer "F.Cu") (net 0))
 (segment (start 78.613 76.708) (end 82.169 76.708) (width 0.15) (layer "F.Cu") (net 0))
 (segment (start 92.837 73.66) (end 97.79 73.66) (width 0.15) (layer "F.Cu") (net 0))
 (segment (start 75.057 87.503) (end 75.057 88.9) (width 0.15) (layer "F.Cu") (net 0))
 (segment (start 70.358 76.835) (end 70.358 74.041) (width 0.15) (layer "F.Cu") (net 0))
 (segment (start 58.42 104.14) (end 48.26 104.14) (width 0.25) (layer "F.Cu") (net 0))
 (segment (start 43.18 66.04) (end 66.04 66.04) (width 0.25) (layer "F.Cu") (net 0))
 (segment (start 70.358 74.041) (end 69.977 73.66) (width 0.15) (layer "F.Cu") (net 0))
 (segment (start 78.613 75.184) (end 80.137 73.66) (width 0.15) (layer "F.Cu") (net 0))
 (segment (start 58.42 63.5) (end 67.31 63.5) (width 0.25) (layer "F.Cu") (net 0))
 (segment (start 92.837 75.057) (end 92.837 73.66) (width 0.25) (layer "F.Cu") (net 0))
 (segment (start 85.795 80.756) (end 85.795 81.256) (width 0.15) (layer "F.Cu") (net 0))
 (segment (start 74.295 80.356) (end 74.295 79.756) (width 0.15) (layer "F.Cu") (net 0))
 (segment (start 82.169 76.708) (end 85.217 73.66) (width 0.15) (layer "F.Cu") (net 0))
 (segment (start 79.295 79.356) (end 79.295 77.931) (width 0.15) (layer "F.Cu") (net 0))
 (segment (start 71.12 99.06) (end 63.5 99.06) (width 0.25) (layer "F.Cu") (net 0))
 (segment (start 88.9 106.68) (end 41.142056 106.68) (width 0.25) (layer "F.Cu") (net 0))
 (segment (start 80.095 80.814) (end 76.073 84.836) (width 0.15) (layer "F.Cu") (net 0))
 (segment (start 80.01 88.773) (end 80.137 88.9) (width 0.15) (layer "F.Cu") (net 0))
 (segment (start 75.184 73.787) (end 75.057 73.66) (width 0.15) (layer "F.Cu") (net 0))
 (segment (start 109.22 71.12) (end 109.22 73.66) (width 0.25) (layer "F.Cu") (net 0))
 (segment (start 90.297 66.167) (end 90.297 73.66) (width 0.25) (layer "F.Cu") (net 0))
 (segment (start 73.295 81.356) (end 74.295 80.356) (width 0.15) (layer "F.Cu") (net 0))
 (segment (start 70.739 85.725) (end 69.977 86.487) (width 0.15) (layer "F.Cu") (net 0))
 (segment (start 76.073 84.836) (end 66.167 84.836) (width 0.15) (layer "F.Cu") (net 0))
 (segment (start 71.12 60.96) (end 74.93 60.96) (width 0.25) (layer "F.Cu") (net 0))
 (segment (start 77.851 75.184) (end 78.613 75.184) (width 0.15) (layer "F.Cu") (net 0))
 (segment (start 58.42 63.5) (end 58.42 58.42) (width 0.25) (layer "F.Cu") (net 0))
 (segment (start 69.85 45.72) (end 74.93 45.72) (width 0.25) (layer "F.Cu") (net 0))
 (segment (start 60.96 43.18) (end 63.5 40.64) (width 0.25) (layer "F.Cu") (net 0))
 (segment (start 79.695 78.293) (end 79.883 78.105) (width 0.15) (layer "F.Cu") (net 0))
 (segment (start 76.895 79.356) (end 76.895 77.022) (width 0.15) (layer "F.Cu") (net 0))
 (segment (start 43.18 66.04) (end 38.1 71.12) (width 0.25) (layer "F.Cu") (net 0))
 (segment (start 72.517 86.741) (end 72.517 88.9) (width 0.15) (layer "F.Cu") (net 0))
 (segment (start 76.2 76.327) (end 75.184 76.327) (width 0.15) (layer "F.Cu") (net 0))
 (segment (start 69.85 63.5) (end 69.85 64.77) (width 0.25) (layer "F.Cu") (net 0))
 (segment (start 76.495 77.216) (end 76.454 77.216) (width 0.15) (layer "F.Cu") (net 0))
 (segment (start 78.095 76.591) (end 78.486 76.2) (width 0.15) (layer "F.Cu") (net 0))
 (via (at 77.597 71.12) (size 0.6) (drill 0.3) (layers "F.Cu" "B.Cu") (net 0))
 (via (at 69.85 63.5) (size 0.6) (drill 0.3) (layers "F.Cu" "B.Cu") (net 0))
 (via (at 58.81 40.64) (size 0.6) (drill 0.3) (layers "F.Cu" "B.Cu") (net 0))
 (via (at 87.757 87.122) (size 0.61) (drill 0.305) (layers "F.Cu" "B.Cu") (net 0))
 (via (at 99.06 60.96) (size 0.6) (drill 0.3) (layers "F.Cu" "B.Cu") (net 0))
 (via (at 67.31 63.5) (size 0.6) (drill 0.3) (layers "F.Cu" "B.Cu") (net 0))
 (via (at 83.566 81.28) (size 0.61) (drill 0.305) (layers "F.Cu" "B.Cu") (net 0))
 (via (at 72.39 66.04) (size 0.6) (drill 0.3) (layers "F.Cu" "B.Cu") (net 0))
 (via (at 60.96 48.26) (size 0.8) (drill 0.4) (layers "F.Cu" "B.Cu") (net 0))
 (via (at 83.566 85.979) (size 0.61) (drill 0.305) (layers "F.Cu" "B.Cu") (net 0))
 (via (at 60.96 43.18) (size 0.8) (drill 0.4) (layers "F.Cu" "B.Cu") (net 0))
 (via (at 83.82 58.42) (size 0.6) (drill 0.3) (layers "F.Cu" "B.Cu") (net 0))
 (via (at 96.52 60.96) (size 0.6) (drill 0.3) (layers "F.Cu" "B.Cu") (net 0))
 (via (at 48.26 68.58) (size 0.6) (drill 0.3) (layers "F.Cu" "B.Cu") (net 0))
 (via (at 48.26 63.5) (size 0.6) (drill 0.3) (layers "F.Cu" "B.Cu") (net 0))
 (via (at 76.327 81.661) (size 0.61) (drill 0.305) (layers "F.Cu" "B.Cu") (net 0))
 (via (at 106.68 58.42) (size 0.6) (drill 0.3) (layers "F.Cu" "B.Cu") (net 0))
 (via (at 90.17 66.04) (size 0.6) (drill 0.3) (layers "F.Cu" "B.Cu") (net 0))
 (via (at 60.96 43.18) (size 0.8) (drill 0.4) (layers "F.Cu" "B.Cu") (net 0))
 (via (at 106.68 66.04) (size 0.6) (drill 0.3) (layers "F.Cu" "B.Cu") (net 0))
 (via (at 60.96 48.26) (size 0.8) (drill 0.4) (layers "F.Cu" "B.Cu") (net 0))
 (via (at 43.18 101.6) (size 0.6) (drill 0.3) (layers "F.Cu" "B.Cu") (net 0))
 (via (at 74.93 60.96) (size 0.6) (drill 0.3) (layers "F.Cu" "B.Cu") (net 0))
 (via (at 90.17 60.96) (size 0.6) (drill 0.3) (layers "F.Cu" "B.Cu") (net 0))
 (segment (start 45.72 55.88) (end 50.8 55.88) (width 0.25) (layer "B.Cu") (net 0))
 (segment (start 106.68 66.04) (end 104.14 68.58) (width 0.25) (layer "B.Cu") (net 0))
 (segment (start 83.947 75.692) (end 84.963 76.708) (width 0.15) (layer "B.Cu") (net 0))
 (segment (start 78.74 69.977) (end 78.74 55.88) (width 0.25) (layer "B.Cu") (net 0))
 (segment (start 67.31 63.5) (end 69.85 63.5) (width 0.25) (layer "B.Cu") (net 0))
 (segment (start 75.565 75.692) (end 83.947 75.692) (width 0.15) (layer "B.Cu") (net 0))
 (segment (start 77.216 87.122) (end 87.757 87.122) (width 0.15) (layer "B.Cu") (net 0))
 (segment (start 83.82 58.42) (end 106.68 58.42) (width 0.25) (layer "B.Cu") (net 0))
 (segment (start 77.597 71.12) (end 78.74 69.977) (width 0.25) (layer "B.Cu") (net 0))
 (segment (start 58.81 38.1) (end 58.81 40.64) (width 0.25) (layer "B.Cu") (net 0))
 (segment (start 90.17 60.96) (end 90.17 66.04) (width 0.25) (layer "B.Cu") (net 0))
 (segment (start 78.74 57.15) (end 78.74 55.88) (width 0.25) (layer "B.Cu") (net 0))
 (segment (start 66.04 55.88) (end 78.74 55.88) (width 0.25) (layer "B.Cu") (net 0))
 (segment (start 60.96 48.26) (end 60.96 43.18) (width 0.25) (layer "B.Cu") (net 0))
 (segment (start 83.566 85.979) (end 83.566 81.28) (width 0.15) (layer "B.Cu") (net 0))
 (segment (start 84.963 76.708) (end 84.795 76.876) (width 0.15) (layer "B.Cu") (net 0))
 (segment (start 99.06 60.96) (end 96.52 60.96) (width 0.25) (layer "B.Cu") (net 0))
 (segment (start 74.295 76.962) (end 75.565 75.692) (width 0.15) (layer "B.Cu") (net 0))
 (segment (start 66.04 38.1) (end 58.81 38.1) (width 0.25) (layer "B.Cu") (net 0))
 (segment (start 80.137 68.58) (end 77.597 71.12) (width 0.25) (layer "B.Cu") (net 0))
 (segment (start 74.295 79.756) (end 74.295 76.962) (width 0.15) (layer "B.Cu") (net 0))
 (segment (start 50.8 93.98) (end 43.18 101.6) (width 0.25) (layer "B.Cu") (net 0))
 (segment (start 84.795 76.876) (end 84.795 79.756) (width 0.15) (layer "B.Cu") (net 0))
 (segment (start 50.8 55.88) (end 50.8 93.98) (width 0.25) (layer "B.Cu") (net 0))
 (segment (start 74.93 60.96) (end 72.39 63.5) (width 0.25) (layer "B.Cu") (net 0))
 (segment (start 43.18 45.72) (end 45.72 45.72) (width 0.25) (layer "B.Cu") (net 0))
 (segment (start 66.04 38.1) (end 66.04 55.88) (width 0.25) (layer "B.Cu") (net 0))
 (segment (start 76.327 86.233) (end 77.216 87.122) (width 0.15) (layer "B.Cu") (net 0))
 (segment (start 104.14 68.58) (end 80.137 68.58) (width 0.25) (layer "B.Cu") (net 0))
 (segment (start 48.26 63.5) (end 48.26 68.58) (width 0.25) (layer "B.Cu") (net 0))
 (segment (start 45.72 45.72) (end 45.72 55.88) (width 0.25) (layer "B.Cu") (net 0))
 (segment (start 72.39 63.5) (end 72.39 66.04) (width 0.25) (layer "B.Cu") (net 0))
 (segment (start 76.327 81.661) (end 76.327 86.233) (width 0.15) (layer "B.Cu") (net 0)))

